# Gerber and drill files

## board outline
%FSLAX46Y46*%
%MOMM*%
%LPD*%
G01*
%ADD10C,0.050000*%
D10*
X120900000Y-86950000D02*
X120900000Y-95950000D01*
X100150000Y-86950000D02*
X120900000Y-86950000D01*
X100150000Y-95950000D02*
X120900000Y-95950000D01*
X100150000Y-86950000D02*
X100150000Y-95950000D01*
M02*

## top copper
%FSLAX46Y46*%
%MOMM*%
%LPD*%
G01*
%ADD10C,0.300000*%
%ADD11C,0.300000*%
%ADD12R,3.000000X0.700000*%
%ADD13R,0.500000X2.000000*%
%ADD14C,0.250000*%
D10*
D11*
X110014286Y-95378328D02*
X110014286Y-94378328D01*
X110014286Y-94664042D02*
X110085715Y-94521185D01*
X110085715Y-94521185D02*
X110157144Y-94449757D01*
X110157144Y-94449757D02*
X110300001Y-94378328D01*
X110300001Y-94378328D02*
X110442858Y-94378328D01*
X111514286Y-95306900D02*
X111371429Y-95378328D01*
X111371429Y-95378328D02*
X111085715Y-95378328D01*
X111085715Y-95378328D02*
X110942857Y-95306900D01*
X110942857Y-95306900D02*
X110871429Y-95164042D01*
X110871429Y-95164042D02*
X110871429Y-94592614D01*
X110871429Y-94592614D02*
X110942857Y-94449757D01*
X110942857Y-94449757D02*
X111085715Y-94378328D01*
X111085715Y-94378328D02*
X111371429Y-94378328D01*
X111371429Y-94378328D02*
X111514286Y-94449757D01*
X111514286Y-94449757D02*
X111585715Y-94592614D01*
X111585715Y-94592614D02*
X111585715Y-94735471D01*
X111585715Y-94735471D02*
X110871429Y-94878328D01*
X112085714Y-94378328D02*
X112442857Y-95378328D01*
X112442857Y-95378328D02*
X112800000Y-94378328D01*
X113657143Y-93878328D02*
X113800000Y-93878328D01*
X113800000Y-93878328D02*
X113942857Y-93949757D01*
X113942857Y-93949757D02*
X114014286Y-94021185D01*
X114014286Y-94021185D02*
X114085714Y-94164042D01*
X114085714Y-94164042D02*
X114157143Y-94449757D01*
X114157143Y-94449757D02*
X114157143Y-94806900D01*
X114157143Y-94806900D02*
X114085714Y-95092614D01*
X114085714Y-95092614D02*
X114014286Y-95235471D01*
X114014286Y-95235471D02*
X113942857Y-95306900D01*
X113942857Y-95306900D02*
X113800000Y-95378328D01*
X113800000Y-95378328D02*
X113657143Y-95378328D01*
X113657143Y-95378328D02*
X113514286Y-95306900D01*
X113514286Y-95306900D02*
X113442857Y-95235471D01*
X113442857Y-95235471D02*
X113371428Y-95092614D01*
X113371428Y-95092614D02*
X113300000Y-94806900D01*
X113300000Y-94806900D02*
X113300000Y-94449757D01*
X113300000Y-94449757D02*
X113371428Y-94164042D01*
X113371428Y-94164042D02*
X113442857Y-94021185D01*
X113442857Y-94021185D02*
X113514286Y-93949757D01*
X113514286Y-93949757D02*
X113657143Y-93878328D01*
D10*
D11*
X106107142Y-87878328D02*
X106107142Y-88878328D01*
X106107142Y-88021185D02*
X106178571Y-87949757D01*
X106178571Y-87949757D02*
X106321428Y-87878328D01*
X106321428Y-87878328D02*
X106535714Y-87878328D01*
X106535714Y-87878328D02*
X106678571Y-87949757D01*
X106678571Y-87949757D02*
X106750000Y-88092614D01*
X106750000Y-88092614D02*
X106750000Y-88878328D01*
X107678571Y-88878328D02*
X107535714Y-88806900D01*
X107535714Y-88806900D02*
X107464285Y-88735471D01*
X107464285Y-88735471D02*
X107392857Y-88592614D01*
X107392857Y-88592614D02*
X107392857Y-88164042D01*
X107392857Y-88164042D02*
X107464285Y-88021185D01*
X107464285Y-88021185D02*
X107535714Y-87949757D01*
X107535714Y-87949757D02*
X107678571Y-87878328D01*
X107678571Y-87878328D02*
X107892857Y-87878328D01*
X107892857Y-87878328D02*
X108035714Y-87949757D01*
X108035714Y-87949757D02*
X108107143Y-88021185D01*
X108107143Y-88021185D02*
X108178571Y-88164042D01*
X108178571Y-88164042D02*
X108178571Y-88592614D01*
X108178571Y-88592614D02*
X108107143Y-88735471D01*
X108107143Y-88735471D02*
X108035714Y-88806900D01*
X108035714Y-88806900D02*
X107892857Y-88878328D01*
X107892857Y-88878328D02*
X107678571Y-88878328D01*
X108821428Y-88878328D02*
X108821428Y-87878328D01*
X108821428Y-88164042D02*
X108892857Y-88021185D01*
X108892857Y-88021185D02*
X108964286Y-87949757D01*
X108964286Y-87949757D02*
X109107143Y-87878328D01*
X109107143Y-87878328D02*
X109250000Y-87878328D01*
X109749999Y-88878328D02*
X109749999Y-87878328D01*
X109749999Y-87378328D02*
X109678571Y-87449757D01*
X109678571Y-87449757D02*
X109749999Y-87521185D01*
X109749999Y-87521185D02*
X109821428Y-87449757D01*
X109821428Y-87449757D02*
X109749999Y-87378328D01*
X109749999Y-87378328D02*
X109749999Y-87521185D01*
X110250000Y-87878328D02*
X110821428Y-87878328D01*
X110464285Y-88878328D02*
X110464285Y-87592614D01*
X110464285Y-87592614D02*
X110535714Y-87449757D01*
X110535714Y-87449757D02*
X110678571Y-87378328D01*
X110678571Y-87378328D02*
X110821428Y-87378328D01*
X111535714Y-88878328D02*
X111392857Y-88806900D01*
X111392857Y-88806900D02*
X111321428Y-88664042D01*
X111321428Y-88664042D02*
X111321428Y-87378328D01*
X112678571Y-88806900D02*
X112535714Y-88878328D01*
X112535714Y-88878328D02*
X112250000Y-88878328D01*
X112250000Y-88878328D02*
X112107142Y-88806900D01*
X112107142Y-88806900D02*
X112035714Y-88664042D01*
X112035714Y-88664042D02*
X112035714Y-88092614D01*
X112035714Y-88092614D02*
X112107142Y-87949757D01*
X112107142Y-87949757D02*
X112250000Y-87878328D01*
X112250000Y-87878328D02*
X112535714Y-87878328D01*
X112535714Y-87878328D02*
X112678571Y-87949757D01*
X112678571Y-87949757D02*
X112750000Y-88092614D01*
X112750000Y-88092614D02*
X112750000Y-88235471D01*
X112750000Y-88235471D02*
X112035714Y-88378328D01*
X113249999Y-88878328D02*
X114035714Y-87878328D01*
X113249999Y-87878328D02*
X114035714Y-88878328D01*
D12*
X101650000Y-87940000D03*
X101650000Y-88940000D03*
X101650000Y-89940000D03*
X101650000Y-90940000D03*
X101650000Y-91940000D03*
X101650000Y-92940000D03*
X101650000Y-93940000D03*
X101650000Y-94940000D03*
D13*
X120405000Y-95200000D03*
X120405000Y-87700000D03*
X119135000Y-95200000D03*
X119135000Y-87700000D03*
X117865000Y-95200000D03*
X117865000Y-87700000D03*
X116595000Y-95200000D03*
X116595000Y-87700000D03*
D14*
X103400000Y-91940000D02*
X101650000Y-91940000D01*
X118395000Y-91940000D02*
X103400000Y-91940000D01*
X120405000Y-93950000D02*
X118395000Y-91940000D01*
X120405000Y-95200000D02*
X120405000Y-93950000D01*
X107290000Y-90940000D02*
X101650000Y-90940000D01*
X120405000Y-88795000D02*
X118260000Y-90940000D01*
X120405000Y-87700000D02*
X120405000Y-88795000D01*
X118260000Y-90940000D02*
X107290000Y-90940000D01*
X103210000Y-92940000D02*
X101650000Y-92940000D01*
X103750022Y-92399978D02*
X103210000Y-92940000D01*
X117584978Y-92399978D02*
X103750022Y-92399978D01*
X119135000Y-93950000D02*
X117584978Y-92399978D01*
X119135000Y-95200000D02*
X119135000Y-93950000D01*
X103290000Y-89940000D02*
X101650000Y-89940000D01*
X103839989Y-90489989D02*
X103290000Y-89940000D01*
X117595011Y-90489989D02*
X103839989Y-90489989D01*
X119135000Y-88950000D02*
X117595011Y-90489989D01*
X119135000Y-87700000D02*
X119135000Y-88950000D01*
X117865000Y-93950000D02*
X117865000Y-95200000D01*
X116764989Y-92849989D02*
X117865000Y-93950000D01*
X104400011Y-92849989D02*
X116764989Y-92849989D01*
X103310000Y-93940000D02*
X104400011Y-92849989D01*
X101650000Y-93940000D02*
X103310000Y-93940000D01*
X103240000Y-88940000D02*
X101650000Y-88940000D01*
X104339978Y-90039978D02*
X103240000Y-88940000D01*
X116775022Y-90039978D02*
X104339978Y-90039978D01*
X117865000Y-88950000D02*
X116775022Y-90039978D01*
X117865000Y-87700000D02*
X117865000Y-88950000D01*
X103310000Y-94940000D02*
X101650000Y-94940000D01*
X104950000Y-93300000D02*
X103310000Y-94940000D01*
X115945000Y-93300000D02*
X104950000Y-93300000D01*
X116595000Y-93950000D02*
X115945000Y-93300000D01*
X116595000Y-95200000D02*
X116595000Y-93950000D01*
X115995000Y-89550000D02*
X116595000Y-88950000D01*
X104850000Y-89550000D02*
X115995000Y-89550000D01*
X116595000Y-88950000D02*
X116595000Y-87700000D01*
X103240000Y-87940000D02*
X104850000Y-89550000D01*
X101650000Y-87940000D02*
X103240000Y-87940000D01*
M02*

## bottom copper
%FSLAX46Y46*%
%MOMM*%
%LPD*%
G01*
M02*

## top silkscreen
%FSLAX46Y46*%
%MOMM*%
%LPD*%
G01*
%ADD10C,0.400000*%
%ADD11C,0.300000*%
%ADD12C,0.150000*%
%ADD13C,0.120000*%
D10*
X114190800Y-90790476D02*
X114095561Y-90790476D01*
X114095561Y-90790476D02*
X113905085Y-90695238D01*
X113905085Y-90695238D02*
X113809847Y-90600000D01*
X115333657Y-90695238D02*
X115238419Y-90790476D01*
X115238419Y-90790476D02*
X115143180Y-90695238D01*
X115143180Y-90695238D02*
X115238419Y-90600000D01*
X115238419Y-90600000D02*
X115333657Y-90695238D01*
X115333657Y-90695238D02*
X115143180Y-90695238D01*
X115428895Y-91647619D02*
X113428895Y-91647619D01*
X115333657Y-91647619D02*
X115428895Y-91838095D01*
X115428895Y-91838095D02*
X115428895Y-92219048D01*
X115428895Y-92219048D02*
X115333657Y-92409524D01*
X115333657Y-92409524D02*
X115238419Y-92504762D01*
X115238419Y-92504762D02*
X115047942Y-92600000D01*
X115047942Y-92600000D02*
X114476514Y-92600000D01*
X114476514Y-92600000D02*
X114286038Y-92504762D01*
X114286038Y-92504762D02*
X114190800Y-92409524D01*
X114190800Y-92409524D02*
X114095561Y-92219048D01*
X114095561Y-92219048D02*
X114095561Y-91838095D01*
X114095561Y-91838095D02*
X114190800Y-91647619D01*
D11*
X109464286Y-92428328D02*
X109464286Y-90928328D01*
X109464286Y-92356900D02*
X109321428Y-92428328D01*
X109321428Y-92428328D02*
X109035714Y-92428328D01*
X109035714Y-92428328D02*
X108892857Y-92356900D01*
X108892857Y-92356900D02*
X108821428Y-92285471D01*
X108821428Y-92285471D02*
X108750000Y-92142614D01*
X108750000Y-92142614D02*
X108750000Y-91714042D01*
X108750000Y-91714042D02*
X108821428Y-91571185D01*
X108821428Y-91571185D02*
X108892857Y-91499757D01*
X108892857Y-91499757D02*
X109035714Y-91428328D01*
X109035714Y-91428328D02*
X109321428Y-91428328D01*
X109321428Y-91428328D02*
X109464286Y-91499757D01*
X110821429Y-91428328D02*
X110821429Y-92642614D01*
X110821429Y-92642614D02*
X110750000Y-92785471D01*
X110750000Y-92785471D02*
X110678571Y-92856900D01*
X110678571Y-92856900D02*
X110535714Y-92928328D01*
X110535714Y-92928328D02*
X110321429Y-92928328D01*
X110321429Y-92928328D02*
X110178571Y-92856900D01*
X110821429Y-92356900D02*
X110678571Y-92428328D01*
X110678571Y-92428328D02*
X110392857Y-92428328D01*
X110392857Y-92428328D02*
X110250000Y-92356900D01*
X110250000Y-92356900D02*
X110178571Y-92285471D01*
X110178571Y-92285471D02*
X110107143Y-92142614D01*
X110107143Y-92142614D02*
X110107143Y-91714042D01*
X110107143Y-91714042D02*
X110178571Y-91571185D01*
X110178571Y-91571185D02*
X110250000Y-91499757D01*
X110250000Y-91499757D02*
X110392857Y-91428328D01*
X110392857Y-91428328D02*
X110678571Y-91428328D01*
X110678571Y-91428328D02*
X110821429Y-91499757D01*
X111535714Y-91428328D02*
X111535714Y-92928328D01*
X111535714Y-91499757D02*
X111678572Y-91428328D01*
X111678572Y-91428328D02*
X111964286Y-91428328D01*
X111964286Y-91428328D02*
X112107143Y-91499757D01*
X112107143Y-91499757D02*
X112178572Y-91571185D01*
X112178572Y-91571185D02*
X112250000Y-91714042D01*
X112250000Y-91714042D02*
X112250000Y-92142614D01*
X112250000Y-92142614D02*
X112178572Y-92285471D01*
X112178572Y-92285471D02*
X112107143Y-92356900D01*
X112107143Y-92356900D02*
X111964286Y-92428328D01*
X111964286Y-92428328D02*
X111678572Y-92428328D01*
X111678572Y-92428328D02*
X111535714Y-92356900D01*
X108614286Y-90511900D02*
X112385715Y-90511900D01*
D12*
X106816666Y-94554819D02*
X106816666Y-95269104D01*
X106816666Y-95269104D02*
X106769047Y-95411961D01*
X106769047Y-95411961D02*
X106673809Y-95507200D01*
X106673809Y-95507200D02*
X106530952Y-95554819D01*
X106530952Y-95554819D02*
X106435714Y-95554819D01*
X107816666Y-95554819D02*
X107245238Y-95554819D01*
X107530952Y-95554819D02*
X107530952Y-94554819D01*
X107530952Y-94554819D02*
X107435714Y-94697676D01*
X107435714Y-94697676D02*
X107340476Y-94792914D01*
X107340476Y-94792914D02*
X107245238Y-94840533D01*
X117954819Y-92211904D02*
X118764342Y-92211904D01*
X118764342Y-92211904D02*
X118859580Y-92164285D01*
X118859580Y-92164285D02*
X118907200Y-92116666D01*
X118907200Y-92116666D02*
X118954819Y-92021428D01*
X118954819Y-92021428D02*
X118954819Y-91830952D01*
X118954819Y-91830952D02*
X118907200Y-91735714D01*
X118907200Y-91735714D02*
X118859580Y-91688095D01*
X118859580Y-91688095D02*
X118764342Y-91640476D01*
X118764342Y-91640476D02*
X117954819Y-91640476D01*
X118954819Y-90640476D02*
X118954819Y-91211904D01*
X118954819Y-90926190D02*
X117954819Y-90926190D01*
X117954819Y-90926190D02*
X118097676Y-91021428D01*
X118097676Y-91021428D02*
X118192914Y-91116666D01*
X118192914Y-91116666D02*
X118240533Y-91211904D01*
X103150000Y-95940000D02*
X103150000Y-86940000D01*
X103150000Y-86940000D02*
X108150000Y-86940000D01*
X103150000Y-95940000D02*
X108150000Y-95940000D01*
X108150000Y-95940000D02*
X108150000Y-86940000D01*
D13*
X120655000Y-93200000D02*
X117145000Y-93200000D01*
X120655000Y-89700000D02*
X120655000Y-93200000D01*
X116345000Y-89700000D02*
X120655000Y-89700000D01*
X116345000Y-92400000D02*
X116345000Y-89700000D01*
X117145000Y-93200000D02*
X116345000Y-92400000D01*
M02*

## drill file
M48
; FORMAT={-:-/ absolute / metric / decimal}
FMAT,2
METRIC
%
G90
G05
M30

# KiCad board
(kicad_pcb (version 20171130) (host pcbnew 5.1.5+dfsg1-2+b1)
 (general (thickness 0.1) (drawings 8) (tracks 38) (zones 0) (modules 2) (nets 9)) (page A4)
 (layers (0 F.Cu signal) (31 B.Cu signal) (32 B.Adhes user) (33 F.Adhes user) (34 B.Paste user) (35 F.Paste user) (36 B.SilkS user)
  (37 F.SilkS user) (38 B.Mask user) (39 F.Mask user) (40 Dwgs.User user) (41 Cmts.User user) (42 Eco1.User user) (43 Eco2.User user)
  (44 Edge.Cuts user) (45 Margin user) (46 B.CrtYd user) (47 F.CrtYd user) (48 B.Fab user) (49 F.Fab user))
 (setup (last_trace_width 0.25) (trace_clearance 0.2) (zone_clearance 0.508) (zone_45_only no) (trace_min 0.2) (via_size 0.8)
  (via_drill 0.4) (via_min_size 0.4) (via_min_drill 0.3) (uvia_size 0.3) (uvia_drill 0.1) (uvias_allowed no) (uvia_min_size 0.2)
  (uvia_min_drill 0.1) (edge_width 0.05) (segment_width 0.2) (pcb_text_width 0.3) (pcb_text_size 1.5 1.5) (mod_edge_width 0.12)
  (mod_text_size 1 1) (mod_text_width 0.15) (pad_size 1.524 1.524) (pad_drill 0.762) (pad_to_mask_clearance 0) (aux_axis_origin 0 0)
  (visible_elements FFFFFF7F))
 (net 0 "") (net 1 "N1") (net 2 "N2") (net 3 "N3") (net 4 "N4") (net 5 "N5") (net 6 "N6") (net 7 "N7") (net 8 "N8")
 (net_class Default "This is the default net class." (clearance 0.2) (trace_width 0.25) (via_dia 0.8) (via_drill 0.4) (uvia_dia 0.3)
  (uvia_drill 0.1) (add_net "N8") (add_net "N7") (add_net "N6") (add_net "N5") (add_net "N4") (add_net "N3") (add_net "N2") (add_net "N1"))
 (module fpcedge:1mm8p (layer F.Cu) (at 103.15 91.44 180)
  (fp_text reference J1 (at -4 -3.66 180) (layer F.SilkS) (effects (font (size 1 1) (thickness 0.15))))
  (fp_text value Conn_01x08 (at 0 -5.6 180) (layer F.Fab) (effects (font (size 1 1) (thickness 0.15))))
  (fp_line (start 0 -4.5) (end 0 4.5) (layer F.SilkS) (width 0.15))
  (fp_line (start 0 4.5) (end -5 4.5) (layer F.SilkS) (width 0.15))
  (fp_line (start 0 -4.5) (end -5 -4.5) (layer F.SilkS) (width 0.15))
  (fp_line (start -5 -4.5) (end -5 4.5) (layer F.SilkS) (width 0.15))
  (pad 8 smd rect (at 1.5 3.5 90) (size 0.7 3) (layers F.Cu F.Paste F.Mask) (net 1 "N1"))
  (pad 7 smd rect (at 1.5 2.5 90) (size 0.7 3) (layers F.Cu F.Paste F.Mask) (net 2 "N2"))
  (pad 6 smd rect (at 1.5 1.5 90) (size 0.7 3) (layers F.Cu F.Paste F.Mask) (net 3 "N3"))
  (pad 5 smd rect (at 1.5 0.5 90) (size 0.7 3) (layers F.Cu F.Paste F.Mask) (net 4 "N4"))
  (pad 4 smd rect (at 1.5 -0.5 90) (size 0.7 3) (layers F.Cu F.Paste F.Mask) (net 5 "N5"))
  (pad 3 smd rect (at 1.5 -1.5 90) (size 0.7 3) (layers F.Cu F.Paste F.Mask) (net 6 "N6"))
  (pad 2 smd rect (at 1.5 -2.5 90) (size 0.7 3) (layers F.Cu F.Paste F.Mask) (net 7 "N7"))
  (pad 1 smd rect (at 1.5 -3.5 90) (size 0.7 3) (layers F.Cu F.Paste F.Mask) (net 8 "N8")))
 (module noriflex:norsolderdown (layer F.Cu) (at 118.5 91.45)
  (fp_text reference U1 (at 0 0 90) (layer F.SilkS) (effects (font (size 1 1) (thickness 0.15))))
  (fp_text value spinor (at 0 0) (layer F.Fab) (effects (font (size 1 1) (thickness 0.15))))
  (fp_line (start 2.155 1.75) (end -1.355 1.75) (layer F.SilkS) (width 0.12))
  (fp_line (start 2.155 -1.75) (end 2.155 1.75) (layer F.SilkS) (width 0.12))
  (fp_line (start -2.155 -1.75) (end 2.155 -1.75) (layer F.SilkS) (width 0.12))
  (fp_line (start -2.155 0.95) (end -2.155 -1.75) (layer F.SilkS) (width 0.12))
  (fp_line (start -1.355 1.75) (end -2.155 0.95) (layer F.SilkS) (width 0.12))
  (pad 4 smd rect (at 1.905 3.75) (size 0.5 2) (layers F.Cu F.Paste F.Mask) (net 5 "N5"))
  (pad 5 smd rect (at 1.905 -3.75) (size 0.5 2) (layers F.Cu F.Paste F.Mask) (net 4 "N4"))
  (pad 3 smd rect (at 0.635 3.75) (size 0.5 2) (layers F.Cu F.Paste F.Mask) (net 6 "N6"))
  (pad 6 smd rect (at 0.635 -3.75) (size 0.5 2) (layers F.Cu F.Paste F.Mask) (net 3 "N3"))
  (pad 2 smd rect (at -0.635 3.75) (size 0.5 2) (layers F.Cu F.Paste F.Mask) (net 7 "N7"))
  (pad 7 smd rect (at -0.635 -3.75) (size 0.5 2) (layers F.Cu F.Paste F.Mask) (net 2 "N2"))
  (pad 1 smd rect (at -1.905 3.75) (size 0.5 2) (layers F.Cu F.Paste F.Mask) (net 8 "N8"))
  (pad 8 smd rect (at -1.905 -3.75) (size 0.5 2) (layers F.Cu F.Paste F.Mask) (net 1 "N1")))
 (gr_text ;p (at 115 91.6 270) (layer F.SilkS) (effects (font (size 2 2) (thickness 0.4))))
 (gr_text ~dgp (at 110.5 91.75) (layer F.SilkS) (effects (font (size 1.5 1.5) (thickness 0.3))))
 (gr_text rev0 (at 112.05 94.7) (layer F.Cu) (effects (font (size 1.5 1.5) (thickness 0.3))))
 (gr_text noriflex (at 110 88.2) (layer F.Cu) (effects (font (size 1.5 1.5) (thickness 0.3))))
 (gr_line (start 120.9 86.95) (end 120.9 95.95) (layer Edge.Cuts) (width 0.05))
 (gr_line (start 100.15 86.95) (end 120.9 86.95) (layer Edge.Cuts) (width 0.05))
 (gr_line (start 100.15 95.95) (end 120.9 95.95) (layer Edge.Cuts) (width 0.05))
 (gr_line (start 100.15 86.95) (end 100.15 95.95) (layer Edge.Cuts) (width 0.05))
 (segment (start 103.4 91.94) (end 101.65 91.94) (width 0.25) (layer F.Cu) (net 5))
 (segment (start 118.395 91.94) (end 103.4 91.94) (width 0.25) (layer F.Cu) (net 5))
 (segment (start 120.405 93.95) (end 118.395 91.94) (width 0.25) (layer F.Cu) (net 5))
 (segment (start 120.405 95.2) (end 120.405 93.95) (width 0.25) (layer F.Cu) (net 5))
 (segment (start 107.29 90.94) (end 101.65 90.94) (width 0.25) (layer F.Cu) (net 4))
 (segment (start 120.405 88.795) (end 118.26 90.94) (width 0.25) (layer F.Cu) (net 4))
 (segment (start 120.405 87.7) (end 120.405 88.795) (width 0.25) (layer F.Cu) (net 4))
 (segment (start 118.26 90.94) (end 107.29 90.94) (width 0.25) (layer F.Cu) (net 4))
 (segment (start 103.21 92.94) (end 101.65 92.94) (width 0.25) (layer F.Cu) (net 6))
 (segment (start 103.750022 92.399978) (end 103.21 92.94) (width 0.25) (layer F.Cu) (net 6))
 (segment (start 117.584978 92.399978) (end 103.750022 92.399978) (width 0.25) (layer F.Cu) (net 6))
 (segment (start 119.135 93.95) (end 117.584978 92.399978) (width 0.25) (layer F.Cu) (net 6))
 (segment (start 119.135 95.2) (end 119.135 93.95) (width 0.25) (layer F.Cu) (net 6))
 (segment (start 103.29 89.94) (end 101.65 89.94) (width 0.25) (layer F.Cu) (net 3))
 (segment (start 103.839989 90.489989) (end 103.29 89.94) (width 0.25) (layer F.Cu) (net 3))
 (segment (start 117.595011 90.489989) (end 103.839989 90.489989) (width 0.25) (layer F.Cu) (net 3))
 (segment (start 119.135 88.95) (end 117.595011 90.489989) (width 0.25) (layer F.Cu) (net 3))
 (segment (start 119.135 87.7) (end 119.135 88.95) (width 0.25) (layer F.Cu) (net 3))
 (segment (start 117.865 93.95) (end 117.865 95.2) (width 0.25) (layer F.Cu) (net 7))
 (segment (start 116.764989 92.849989) (end 117.865 93.95) (width 0.25) (layer F.Cu) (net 7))
 (segment (start 104.400011 92.849989) (end 116.764989 92.849989) (width 0.25) (layer F.Cu) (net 7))
 (segment (start 103.31 93.94) (end 104.400011 92.849989) (width 0.25) (layer F.Cu) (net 7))
 (segment (start 101.65 93.94) (end 103.31 93.94) (width 0.25) (layer F.Cu) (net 7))
 (segment (start 103.24 88.94) (end 101.65 88.94) (width 0.25) (layer F.Cu) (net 2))
 (segment (start 104.339978 90.039978) (end 103.24 88.94) (width 0.25) (layer F.Cu) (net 2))
 (segment (start 116.775022 90.039978) (end 104.339978 90.039978) (width 0.25) (layer F.Cu) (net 2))
 (segment (start 117.865 88.95) (end 116.775022 90.039978) (width 0.25) (layer F.Cu) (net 2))
 (segment (start 117.865 87.7) (end 117.865 88.95) (width 0.25) (layer F.Cu) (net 2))
 (segment (start 103.31 94.94) (end 101.65 94.94) (width 0.25) (layer F.Cu) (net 8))
 (segment (start 104.95 93.3) (end 103.31 94.94) (width 0.25) (layer F.Cu) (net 8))
 (segment (start 115.945 93.3) (end 104.95 93.3) (width 0.25) (layer F.Cu) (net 8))
 (segment (start 116.595 93.95) (end 115.945 93.3) (width 0.25) (layer F.Cu) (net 8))
 (segment (start 116.595 95.2) (end 116.595 93.95) (width 0.25) (layer F.Cu) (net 8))
 (segment (start 115.995 89.55) (end 116.595 88.95) (width 0.25) (layer F.Cu) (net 1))
 (segment (start 104.85 89.55) (end 115.995 89.55) (width 0.25) (layer F.Cu) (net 1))
 (segment (start 116.595 88.95) (end 116.595 87.7) (width 0.25) (layer F.Cu) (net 1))
 (segment (start 103.24 87.94) (end 104.85 89.55) (width 0.25) (layer F.Cu) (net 1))
 (segment (start 101.65 87.94) (end 103.24 87.94) (width 0.25) (layer F.Cu) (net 1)))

